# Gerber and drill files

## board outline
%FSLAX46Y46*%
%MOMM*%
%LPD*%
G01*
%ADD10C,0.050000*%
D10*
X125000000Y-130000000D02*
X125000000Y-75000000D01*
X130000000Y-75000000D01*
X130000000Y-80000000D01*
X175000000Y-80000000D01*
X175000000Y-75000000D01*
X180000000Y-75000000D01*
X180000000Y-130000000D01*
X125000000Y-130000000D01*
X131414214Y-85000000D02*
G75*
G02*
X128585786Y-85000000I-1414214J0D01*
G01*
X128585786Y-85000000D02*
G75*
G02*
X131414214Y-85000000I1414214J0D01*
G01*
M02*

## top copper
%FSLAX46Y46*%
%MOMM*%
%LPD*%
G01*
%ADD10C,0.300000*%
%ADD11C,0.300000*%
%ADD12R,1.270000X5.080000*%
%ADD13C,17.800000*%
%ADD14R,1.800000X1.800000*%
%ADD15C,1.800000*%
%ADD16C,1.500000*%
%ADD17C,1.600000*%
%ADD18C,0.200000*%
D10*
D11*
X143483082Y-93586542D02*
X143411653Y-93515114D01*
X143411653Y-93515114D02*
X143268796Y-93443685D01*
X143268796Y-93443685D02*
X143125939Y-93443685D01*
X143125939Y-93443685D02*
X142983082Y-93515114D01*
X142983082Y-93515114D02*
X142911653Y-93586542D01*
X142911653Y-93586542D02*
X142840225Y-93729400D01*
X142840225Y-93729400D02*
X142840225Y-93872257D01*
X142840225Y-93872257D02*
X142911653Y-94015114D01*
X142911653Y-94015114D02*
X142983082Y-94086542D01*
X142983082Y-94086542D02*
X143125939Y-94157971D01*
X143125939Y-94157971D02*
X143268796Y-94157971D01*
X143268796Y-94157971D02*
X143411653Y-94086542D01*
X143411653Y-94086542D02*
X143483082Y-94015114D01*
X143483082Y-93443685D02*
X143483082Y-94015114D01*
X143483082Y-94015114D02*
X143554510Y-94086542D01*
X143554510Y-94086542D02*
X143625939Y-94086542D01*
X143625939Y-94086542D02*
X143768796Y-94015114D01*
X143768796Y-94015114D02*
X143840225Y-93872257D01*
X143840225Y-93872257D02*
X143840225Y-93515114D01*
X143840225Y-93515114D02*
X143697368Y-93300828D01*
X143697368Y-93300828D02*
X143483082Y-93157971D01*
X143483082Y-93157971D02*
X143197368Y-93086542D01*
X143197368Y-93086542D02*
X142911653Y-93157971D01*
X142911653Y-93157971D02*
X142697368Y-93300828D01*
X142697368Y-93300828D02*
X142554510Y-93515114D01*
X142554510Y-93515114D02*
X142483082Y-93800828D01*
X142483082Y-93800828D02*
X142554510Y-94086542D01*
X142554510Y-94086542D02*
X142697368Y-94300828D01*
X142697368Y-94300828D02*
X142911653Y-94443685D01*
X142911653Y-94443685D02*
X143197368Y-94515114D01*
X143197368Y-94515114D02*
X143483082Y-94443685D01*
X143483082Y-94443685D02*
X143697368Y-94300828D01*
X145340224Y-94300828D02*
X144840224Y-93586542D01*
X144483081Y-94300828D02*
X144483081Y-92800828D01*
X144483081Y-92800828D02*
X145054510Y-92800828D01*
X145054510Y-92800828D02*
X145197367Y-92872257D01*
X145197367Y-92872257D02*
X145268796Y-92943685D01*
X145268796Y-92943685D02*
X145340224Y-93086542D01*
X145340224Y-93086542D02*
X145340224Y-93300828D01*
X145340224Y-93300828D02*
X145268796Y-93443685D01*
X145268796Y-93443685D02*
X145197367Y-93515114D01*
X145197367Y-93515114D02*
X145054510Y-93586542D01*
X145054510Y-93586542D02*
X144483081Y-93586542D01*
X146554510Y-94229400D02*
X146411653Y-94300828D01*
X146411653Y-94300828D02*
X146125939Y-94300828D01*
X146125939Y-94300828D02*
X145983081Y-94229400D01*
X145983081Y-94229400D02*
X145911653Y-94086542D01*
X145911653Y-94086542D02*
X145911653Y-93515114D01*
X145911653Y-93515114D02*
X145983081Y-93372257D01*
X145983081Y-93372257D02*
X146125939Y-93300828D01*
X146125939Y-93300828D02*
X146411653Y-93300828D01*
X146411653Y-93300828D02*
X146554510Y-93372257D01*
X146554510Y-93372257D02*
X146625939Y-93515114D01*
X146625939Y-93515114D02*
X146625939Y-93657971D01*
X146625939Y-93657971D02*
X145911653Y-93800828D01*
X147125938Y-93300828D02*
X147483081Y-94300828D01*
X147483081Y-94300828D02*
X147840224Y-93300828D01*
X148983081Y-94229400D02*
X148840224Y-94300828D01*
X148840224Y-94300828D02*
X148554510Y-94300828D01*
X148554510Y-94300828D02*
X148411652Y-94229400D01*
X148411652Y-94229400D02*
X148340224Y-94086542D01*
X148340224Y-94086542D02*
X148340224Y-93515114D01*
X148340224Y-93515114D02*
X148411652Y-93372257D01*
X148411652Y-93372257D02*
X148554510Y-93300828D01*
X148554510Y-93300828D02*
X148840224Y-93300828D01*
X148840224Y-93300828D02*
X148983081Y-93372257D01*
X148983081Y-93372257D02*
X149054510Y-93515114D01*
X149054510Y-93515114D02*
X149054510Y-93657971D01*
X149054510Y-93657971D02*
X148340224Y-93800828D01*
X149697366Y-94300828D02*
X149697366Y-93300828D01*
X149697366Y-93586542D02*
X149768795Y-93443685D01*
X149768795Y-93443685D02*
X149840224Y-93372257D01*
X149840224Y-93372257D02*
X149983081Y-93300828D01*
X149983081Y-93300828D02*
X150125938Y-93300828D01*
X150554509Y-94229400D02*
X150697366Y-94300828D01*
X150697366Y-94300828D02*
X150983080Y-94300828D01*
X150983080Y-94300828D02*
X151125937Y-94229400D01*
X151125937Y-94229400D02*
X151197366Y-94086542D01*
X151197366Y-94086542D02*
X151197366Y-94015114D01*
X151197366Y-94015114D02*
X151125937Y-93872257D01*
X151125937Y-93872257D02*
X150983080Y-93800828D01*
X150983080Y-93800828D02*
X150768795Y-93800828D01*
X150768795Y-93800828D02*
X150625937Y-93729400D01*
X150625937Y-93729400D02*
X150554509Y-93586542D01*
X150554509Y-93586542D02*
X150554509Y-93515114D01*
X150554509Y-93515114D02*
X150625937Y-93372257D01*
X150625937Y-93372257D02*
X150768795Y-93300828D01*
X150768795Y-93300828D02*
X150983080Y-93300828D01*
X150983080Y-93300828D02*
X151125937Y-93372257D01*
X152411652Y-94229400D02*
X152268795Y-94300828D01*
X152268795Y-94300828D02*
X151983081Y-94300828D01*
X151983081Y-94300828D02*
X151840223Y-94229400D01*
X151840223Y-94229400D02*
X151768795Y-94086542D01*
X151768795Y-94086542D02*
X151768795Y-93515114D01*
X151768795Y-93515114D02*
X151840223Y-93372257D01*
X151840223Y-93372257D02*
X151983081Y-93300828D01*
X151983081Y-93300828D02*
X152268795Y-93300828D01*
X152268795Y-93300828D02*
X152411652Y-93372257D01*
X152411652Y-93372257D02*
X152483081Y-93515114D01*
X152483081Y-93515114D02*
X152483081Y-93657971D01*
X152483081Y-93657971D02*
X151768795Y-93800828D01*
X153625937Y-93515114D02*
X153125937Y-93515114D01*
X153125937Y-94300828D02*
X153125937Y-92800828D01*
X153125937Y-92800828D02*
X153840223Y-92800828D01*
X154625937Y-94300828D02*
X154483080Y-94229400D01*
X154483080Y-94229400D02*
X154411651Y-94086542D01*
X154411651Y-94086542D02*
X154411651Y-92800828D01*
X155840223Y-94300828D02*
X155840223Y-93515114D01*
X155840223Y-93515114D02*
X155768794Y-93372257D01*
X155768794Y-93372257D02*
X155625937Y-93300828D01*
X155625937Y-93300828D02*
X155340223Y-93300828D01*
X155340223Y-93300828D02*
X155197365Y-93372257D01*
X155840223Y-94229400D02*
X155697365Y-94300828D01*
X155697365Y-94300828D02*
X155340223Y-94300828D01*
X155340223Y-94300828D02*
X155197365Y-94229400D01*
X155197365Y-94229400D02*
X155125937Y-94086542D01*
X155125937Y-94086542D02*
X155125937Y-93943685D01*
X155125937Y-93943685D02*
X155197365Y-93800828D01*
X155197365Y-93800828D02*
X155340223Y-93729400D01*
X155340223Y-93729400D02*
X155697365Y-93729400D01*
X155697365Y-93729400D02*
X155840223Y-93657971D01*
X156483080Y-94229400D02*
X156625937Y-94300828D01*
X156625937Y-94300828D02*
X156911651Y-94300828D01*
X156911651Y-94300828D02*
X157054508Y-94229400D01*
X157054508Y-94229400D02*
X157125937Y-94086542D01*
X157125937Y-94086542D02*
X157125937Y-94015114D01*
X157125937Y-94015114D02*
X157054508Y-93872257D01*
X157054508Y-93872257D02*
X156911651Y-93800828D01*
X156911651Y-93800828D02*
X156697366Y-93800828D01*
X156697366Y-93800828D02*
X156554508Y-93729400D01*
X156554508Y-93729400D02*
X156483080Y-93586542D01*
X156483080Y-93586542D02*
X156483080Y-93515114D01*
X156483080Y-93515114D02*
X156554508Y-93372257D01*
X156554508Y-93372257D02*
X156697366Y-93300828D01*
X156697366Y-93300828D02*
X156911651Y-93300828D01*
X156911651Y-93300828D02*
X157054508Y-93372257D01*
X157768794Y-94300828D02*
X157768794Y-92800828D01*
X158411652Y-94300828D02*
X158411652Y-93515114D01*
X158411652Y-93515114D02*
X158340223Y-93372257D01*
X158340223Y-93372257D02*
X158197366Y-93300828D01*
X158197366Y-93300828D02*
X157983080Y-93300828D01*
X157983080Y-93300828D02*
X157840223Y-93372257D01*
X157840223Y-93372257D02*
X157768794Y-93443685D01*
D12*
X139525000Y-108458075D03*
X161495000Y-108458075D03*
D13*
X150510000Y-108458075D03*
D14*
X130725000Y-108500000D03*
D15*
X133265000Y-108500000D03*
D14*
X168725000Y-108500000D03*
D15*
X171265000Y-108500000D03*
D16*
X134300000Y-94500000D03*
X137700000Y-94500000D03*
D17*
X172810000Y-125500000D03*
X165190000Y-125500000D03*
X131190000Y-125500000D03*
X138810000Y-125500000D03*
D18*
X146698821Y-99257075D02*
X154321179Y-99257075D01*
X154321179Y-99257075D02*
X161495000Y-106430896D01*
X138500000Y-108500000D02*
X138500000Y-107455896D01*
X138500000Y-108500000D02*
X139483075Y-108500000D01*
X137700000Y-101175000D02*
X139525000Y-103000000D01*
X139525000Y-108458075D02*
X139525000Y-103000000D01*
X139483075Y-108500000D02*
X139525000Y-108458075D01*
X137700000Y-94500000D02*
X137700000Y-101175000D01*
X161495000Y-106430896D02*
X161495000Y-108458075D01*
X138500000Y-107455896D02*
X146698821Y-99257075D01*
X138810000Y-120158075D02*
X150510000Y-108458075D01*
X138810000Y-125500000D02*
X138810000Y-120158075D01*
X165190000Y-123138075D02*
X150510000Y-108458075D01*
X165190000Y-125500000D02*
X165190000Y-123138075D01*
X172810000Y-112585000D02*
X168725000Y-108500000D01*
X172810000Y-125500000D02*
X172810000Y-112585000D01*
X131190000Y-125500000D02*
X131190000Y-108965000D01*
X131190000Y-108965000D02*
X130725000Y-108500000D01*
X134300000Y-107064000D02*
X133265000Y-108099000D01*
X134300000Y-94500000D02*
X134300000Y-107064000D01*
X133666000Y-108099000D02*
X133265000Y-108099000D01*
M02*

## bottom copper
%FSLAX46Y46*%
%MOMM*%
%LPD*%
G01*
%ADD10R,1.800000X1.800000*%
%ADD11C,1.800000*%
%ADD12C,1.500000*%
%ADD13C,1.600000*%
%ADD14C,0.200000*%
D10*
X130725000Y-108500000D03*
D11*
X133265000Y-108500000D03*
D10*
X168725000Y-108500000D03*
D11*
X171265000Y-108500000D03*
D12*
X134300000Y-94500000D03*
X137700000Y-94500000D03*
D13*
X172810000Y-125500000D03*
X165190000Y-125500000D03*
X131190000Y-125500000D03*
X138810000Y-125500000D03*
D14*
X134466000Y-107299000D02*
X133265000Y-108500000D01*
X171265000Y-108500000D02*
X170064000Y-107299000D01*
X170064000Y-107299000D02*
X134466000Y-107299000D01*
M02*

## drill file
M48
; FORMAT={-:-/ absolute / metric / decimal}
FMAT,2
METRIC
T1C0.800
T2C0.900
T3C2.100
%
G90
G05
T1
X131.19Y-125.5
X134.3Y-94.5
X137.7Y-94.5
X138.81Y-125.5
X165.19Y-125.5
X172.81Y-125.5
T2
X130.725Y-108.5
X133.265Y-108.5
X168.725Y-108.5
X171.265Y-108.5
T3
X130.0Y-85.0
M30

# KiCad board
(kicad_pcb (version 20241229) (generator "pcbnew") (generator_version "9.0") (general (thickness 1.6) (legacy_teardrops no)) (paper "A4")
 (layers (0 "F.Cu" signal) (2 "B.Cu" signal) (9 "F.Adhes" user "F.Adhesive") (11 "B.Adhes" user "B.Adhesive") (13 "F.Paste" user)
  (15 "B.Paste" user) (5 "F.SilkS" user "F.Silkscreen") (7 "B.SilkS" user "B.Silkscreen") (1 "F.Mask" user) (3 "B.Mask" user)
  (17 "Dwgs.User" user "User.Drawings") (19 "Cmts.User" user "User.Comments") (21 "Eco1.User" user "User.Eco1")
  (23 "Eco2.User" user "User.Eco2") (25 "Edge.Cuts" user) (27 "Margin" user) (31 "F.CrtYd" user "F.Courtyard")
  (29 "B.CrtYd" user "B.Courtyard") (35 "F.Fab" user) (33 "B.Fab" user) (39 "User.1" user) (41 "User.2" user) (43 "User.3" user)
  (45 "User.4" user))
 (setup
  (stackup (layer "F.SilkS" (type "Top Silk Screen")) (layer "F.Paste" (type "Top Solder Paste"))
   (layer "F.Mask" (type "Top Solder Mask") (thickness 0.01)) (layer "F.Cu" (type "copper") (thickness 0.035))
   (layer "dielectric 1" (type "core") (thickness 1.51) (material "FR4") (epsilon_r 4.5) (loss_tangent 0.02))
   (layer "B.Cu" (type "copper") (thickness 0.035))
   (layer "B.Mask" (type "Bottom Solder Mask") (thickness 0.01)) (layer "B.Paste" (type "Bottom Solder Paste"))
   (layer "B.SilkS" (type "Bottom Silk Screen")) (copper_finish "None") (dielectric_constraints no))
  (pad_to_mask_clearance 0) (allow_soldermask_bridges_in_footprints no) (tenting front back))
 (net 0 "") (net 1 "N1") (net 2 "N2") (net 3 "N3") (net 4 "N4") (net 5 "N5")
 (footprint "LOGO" (layer "F.Cu") (at 150.5 87)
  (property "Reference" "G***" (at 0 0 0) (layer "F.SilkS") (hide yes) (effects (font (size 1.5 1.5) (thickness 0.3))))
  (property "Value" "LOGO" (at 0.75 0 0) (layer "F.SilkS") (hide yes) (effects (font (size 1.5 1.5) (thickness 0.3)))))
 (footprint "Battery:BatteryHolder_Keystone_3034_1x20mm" (layer "F.Cu") (at 150.51 108.458075)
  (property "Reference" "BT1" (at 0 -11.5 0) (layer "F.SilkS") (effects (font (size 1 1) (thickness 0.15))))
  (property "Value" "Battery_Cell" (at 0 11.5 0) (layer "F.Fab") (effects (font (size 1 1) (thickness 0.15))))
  (pad "1" smd rect (at -10.985 0) (size 1.27 5.08) (layers "F.Cu" "F.Mask" "F.Paste") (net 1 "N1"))
  (pad "1" smd rect (at 10.985 0) (size 1.27 5.08) (layers "F.Cu" "F.Mask" "F.Paste") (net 1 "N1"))
  (pad "2" smd circle (at 0 0) (size 17.8 17.8) (layers "F.Cu" "F.Mask") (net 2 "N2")))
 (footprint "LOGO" (layer "F.Cu") (at 170 90)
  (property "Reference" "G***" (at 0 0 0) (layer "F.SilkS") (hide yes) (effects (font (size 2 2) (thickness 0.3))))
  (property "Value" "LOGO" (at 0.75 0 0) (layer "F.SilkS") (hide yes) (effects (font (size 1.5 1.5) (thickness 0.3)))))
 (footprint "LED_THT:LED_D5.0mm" (layer "F.Cu") (at 130.725 108.5)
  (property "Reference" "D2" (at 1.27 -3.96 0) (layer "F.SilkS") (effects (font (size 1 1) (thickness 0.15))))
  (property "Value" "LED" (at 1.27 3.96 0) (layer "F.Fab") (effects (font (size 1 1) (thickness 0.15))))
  (pad "1" thru_hole rect (at 0 0) (size 1.8 1.8) (drill 0.9) (layers "*.Cu" "*.Mask") (remove_unused_layers no) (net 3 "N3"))
  (pad "2" thru_hole circle (at 2.54 0) (size 1.8 1.8) (drill 0.9) (layers "*.Cu" "*.Mask") (remove_unused_layers no) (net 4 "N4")))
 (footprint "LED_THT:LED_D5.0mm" (layer "F.Cu") (at 168.725 108.5)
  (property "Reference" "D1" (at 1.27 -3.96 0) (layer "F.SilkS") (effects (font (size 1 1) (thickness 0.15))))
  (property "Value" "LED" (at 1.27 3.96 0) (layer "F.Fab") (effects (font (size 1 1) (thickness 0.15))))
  (pad "1" thru_hole rect (at 0 0) (size 1.8 1.8) (drill 0.9) (layers "*.Cu" "*.Mask") (remove_unused_layers no) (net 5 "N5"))
  (pad "2" thru_hole circle (at 2.54 0) (size 1.8 1.8) (drill 0.9) (layers "*.Cu" "*.Mask") (remove_unused_layers no) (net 4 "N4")))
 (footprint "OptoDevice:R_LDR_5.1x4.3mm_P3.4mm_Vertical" (layer "F.Cu") (at 134.3 94.5)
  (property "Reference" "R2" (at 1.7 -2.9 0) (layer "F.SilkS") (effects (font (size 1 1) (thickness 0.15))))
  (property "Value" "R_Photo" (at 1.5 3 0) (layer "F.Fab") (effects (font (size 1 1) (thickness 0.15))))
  (pad "1" thru_hole circle (at 0 0) (size 1.5 1.5) (drill 0.8) (layers "*.Cu" "*.Mask") (remove_unused_layers no) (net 4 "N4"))
  (pad "2" thru_hole circle (at 3.4 0) (size 1.5 1.5) (drill 0.8) (layers "*.Cu" "*.Mask") (remove_unused_layers no) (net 1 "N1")))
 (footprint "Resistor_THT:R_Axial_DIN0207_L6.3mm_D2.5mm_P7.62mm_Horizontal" (layer "F.Cu") (at 172.81 125.5 180)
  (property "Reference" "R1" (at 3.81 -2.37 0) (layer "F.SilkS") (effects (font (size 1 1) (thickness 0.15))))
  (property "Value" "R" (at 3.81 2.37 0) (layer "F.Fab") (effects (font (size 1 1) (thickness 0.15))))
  (pad "1" thru_hole circle (at 0 0 180) (size 1.6 1.6) (drill 0.8) (layers "*.Cu" "*.Mask") (remove_unused_layers no) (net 5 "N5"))
  (pad "2" thru_hole circle (at 7.62 0 180) (size 1.6 1.6) (drill 0.8) (layers "*.Cu" "*.Mask") (remove_unused_layers no) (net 2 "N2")))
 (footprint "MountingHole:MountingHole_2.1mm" (layer "F.Cu") (at 130 85)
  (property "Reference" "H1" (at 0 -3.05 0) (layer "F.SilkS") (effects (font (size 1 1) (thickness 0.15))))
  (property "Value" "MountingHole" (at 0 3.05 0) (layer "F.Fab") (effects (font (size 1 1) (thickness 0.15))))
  (pad "" np_thru_hole circle (at 0 0) (size 2.1 2.1) (drill 2.1) (layers "*.Cu" "*.Mask")))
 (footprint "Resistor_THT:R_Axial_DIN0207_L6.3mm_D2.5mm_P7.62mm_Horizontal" (layer "F.Cu") (at 131.19 125.5)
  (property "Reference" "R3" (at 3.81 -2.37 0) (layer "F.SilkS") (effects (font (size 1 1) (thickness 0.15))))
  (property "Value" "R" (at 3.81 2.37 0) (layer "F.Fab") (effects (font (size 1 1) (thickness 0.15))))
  (pad "1" thru_hole circle (at 0 0) (size 1.6 1.6) (drill 0.8) (layers "*.Cu" "*.Mask") (remove_unused_layers no) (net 3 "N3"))
  (pad "2" thru_hole circle (at 7.62 0) (size 1.6 1.6) (drill 0.8) (layers "*.Cu" "*.Mask") (remove_unused_layers no) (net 2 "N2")))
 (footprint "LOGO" (layer "B.Cu") (at 150 105 180)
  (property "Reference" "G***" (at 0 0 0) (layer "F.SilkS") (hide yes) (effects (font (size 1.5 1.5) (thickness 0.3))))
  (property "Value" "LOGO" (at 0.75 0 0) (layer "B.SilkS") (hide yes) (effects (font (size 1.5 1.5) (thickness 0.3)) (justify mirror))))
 (gr_poly
  (pts (xy 125 130) (xy 125 75) (xy 130 75) (xy 130 80) (xy 175 80) (xy 175 75) (xy 180 75) (xy 180 130)) (stroke (width 0.05) (type solid))
  (fill no) (layer "Edge.Cuts"))
 (gr_circle (center 130 85) (end 131 86) (stroke (width 0.05) (type default)) (fill no) (layer "Edge.Cuts"))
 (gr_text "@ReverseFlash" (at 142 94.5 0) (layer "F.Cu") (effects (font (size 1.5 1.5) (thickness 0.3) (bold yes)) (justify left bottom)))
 (segment (start 146.698821 99.257075) (end 154.321179 99.257075) (width 0.2) (layer "F.Cu") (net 1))
 (segment (start 154.321179 99.257075) (end 161.495 106.430896) (width 0.2) (layer "F.Cu") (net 1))
 (segment (start 138.5 108.5) (end 138.5 107.455896) (width 0.2) (layer "F.Cu") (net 1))
 (segment (start 138.5 108.5) (end 139.483075 108.5) (width 0.2) (layer "F.Cu") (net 1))
 (segment (start 137.7 101.175) (end 139.525 103) (width 0.2) (layer "F.Cu") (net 1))
 (segment (start 139.525 108.458075) (end 139.525 103) (width 0.2) (layer "F.Cu") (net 1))
 (segment (start 139.483075 108.5) (end 139.525 108.458075) (width 0.2) (layer "F.Cu") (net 1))
 (segment (start 137.7 94.5) (end 137.7 101.175) (width 0.2) (layer "F.Cu") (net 1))
 (segment (start 161.495 106.430896) (end 161.495 108.458075) (width 0.2) (layer "F.Cu") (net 1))
 (segment (start 138.5 107.455896) (end 146.698821 99.257075) (width 0.2) (layer "F.Cu") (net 1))
 (segment (start 138.81 120.158075) (end 150.51 108.458075) (width 0.2) (layer "F.Cu") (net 2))
 (segment (start 138.81 125.5) (end 138.81 120.158075) (width 0.2) (layer "F.Cu") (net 2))
 (segment (start 165.19 123.138075) (end 150.51 108.458075) (width 0.2) (layer "F.Cu") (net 2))
 (segment (start 165.19 125.5) (end 165.19 123.138075) (width 0.2) (layer "F.Cu") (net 2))
 (segment (start 172.81 112.585) (end 168.725 108.5) (width 0.2) (layer "F.Cu") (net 5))
 (segment (start 172.81 125.5) (end 172.81 112.585) (width 0.2) (layer "F.Cu") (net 5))
 (segment (start 131.19 125.5) (end 131.19 108.965) (width 0.2) (layer "F.Cu") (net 3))
 (segment (start 131.19 108.965) (end 130.725 108.5) (width 0.2) (layer "F.Cu") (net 3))
 (segment (start 134.3 107.064) (end 133.265 108.099) (width 0.2) (layer "F.Cu") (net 4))
 (segment (start 134.3 94.5) (end 134.3 107.064) (width 0.2) (layer "F.Cu") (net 4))
 (segment (start 133.666 108.099) (end 133.265 108.099) (width 0.2) (layer "F.Cu") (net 4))
 (segment (start 134.466 107.299) (end 133.265 108.5) (width 0.2) (layer "B.Cu") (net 4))
 (segment (start 171.265 108.5) (end 170.064 107.299) (width 0.2) (layer "B.Cu") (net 4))
 (segment (start 170.064 107.299) (end 134.466 107.299) (width 0.2) (layer "B.Cu") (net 4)))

